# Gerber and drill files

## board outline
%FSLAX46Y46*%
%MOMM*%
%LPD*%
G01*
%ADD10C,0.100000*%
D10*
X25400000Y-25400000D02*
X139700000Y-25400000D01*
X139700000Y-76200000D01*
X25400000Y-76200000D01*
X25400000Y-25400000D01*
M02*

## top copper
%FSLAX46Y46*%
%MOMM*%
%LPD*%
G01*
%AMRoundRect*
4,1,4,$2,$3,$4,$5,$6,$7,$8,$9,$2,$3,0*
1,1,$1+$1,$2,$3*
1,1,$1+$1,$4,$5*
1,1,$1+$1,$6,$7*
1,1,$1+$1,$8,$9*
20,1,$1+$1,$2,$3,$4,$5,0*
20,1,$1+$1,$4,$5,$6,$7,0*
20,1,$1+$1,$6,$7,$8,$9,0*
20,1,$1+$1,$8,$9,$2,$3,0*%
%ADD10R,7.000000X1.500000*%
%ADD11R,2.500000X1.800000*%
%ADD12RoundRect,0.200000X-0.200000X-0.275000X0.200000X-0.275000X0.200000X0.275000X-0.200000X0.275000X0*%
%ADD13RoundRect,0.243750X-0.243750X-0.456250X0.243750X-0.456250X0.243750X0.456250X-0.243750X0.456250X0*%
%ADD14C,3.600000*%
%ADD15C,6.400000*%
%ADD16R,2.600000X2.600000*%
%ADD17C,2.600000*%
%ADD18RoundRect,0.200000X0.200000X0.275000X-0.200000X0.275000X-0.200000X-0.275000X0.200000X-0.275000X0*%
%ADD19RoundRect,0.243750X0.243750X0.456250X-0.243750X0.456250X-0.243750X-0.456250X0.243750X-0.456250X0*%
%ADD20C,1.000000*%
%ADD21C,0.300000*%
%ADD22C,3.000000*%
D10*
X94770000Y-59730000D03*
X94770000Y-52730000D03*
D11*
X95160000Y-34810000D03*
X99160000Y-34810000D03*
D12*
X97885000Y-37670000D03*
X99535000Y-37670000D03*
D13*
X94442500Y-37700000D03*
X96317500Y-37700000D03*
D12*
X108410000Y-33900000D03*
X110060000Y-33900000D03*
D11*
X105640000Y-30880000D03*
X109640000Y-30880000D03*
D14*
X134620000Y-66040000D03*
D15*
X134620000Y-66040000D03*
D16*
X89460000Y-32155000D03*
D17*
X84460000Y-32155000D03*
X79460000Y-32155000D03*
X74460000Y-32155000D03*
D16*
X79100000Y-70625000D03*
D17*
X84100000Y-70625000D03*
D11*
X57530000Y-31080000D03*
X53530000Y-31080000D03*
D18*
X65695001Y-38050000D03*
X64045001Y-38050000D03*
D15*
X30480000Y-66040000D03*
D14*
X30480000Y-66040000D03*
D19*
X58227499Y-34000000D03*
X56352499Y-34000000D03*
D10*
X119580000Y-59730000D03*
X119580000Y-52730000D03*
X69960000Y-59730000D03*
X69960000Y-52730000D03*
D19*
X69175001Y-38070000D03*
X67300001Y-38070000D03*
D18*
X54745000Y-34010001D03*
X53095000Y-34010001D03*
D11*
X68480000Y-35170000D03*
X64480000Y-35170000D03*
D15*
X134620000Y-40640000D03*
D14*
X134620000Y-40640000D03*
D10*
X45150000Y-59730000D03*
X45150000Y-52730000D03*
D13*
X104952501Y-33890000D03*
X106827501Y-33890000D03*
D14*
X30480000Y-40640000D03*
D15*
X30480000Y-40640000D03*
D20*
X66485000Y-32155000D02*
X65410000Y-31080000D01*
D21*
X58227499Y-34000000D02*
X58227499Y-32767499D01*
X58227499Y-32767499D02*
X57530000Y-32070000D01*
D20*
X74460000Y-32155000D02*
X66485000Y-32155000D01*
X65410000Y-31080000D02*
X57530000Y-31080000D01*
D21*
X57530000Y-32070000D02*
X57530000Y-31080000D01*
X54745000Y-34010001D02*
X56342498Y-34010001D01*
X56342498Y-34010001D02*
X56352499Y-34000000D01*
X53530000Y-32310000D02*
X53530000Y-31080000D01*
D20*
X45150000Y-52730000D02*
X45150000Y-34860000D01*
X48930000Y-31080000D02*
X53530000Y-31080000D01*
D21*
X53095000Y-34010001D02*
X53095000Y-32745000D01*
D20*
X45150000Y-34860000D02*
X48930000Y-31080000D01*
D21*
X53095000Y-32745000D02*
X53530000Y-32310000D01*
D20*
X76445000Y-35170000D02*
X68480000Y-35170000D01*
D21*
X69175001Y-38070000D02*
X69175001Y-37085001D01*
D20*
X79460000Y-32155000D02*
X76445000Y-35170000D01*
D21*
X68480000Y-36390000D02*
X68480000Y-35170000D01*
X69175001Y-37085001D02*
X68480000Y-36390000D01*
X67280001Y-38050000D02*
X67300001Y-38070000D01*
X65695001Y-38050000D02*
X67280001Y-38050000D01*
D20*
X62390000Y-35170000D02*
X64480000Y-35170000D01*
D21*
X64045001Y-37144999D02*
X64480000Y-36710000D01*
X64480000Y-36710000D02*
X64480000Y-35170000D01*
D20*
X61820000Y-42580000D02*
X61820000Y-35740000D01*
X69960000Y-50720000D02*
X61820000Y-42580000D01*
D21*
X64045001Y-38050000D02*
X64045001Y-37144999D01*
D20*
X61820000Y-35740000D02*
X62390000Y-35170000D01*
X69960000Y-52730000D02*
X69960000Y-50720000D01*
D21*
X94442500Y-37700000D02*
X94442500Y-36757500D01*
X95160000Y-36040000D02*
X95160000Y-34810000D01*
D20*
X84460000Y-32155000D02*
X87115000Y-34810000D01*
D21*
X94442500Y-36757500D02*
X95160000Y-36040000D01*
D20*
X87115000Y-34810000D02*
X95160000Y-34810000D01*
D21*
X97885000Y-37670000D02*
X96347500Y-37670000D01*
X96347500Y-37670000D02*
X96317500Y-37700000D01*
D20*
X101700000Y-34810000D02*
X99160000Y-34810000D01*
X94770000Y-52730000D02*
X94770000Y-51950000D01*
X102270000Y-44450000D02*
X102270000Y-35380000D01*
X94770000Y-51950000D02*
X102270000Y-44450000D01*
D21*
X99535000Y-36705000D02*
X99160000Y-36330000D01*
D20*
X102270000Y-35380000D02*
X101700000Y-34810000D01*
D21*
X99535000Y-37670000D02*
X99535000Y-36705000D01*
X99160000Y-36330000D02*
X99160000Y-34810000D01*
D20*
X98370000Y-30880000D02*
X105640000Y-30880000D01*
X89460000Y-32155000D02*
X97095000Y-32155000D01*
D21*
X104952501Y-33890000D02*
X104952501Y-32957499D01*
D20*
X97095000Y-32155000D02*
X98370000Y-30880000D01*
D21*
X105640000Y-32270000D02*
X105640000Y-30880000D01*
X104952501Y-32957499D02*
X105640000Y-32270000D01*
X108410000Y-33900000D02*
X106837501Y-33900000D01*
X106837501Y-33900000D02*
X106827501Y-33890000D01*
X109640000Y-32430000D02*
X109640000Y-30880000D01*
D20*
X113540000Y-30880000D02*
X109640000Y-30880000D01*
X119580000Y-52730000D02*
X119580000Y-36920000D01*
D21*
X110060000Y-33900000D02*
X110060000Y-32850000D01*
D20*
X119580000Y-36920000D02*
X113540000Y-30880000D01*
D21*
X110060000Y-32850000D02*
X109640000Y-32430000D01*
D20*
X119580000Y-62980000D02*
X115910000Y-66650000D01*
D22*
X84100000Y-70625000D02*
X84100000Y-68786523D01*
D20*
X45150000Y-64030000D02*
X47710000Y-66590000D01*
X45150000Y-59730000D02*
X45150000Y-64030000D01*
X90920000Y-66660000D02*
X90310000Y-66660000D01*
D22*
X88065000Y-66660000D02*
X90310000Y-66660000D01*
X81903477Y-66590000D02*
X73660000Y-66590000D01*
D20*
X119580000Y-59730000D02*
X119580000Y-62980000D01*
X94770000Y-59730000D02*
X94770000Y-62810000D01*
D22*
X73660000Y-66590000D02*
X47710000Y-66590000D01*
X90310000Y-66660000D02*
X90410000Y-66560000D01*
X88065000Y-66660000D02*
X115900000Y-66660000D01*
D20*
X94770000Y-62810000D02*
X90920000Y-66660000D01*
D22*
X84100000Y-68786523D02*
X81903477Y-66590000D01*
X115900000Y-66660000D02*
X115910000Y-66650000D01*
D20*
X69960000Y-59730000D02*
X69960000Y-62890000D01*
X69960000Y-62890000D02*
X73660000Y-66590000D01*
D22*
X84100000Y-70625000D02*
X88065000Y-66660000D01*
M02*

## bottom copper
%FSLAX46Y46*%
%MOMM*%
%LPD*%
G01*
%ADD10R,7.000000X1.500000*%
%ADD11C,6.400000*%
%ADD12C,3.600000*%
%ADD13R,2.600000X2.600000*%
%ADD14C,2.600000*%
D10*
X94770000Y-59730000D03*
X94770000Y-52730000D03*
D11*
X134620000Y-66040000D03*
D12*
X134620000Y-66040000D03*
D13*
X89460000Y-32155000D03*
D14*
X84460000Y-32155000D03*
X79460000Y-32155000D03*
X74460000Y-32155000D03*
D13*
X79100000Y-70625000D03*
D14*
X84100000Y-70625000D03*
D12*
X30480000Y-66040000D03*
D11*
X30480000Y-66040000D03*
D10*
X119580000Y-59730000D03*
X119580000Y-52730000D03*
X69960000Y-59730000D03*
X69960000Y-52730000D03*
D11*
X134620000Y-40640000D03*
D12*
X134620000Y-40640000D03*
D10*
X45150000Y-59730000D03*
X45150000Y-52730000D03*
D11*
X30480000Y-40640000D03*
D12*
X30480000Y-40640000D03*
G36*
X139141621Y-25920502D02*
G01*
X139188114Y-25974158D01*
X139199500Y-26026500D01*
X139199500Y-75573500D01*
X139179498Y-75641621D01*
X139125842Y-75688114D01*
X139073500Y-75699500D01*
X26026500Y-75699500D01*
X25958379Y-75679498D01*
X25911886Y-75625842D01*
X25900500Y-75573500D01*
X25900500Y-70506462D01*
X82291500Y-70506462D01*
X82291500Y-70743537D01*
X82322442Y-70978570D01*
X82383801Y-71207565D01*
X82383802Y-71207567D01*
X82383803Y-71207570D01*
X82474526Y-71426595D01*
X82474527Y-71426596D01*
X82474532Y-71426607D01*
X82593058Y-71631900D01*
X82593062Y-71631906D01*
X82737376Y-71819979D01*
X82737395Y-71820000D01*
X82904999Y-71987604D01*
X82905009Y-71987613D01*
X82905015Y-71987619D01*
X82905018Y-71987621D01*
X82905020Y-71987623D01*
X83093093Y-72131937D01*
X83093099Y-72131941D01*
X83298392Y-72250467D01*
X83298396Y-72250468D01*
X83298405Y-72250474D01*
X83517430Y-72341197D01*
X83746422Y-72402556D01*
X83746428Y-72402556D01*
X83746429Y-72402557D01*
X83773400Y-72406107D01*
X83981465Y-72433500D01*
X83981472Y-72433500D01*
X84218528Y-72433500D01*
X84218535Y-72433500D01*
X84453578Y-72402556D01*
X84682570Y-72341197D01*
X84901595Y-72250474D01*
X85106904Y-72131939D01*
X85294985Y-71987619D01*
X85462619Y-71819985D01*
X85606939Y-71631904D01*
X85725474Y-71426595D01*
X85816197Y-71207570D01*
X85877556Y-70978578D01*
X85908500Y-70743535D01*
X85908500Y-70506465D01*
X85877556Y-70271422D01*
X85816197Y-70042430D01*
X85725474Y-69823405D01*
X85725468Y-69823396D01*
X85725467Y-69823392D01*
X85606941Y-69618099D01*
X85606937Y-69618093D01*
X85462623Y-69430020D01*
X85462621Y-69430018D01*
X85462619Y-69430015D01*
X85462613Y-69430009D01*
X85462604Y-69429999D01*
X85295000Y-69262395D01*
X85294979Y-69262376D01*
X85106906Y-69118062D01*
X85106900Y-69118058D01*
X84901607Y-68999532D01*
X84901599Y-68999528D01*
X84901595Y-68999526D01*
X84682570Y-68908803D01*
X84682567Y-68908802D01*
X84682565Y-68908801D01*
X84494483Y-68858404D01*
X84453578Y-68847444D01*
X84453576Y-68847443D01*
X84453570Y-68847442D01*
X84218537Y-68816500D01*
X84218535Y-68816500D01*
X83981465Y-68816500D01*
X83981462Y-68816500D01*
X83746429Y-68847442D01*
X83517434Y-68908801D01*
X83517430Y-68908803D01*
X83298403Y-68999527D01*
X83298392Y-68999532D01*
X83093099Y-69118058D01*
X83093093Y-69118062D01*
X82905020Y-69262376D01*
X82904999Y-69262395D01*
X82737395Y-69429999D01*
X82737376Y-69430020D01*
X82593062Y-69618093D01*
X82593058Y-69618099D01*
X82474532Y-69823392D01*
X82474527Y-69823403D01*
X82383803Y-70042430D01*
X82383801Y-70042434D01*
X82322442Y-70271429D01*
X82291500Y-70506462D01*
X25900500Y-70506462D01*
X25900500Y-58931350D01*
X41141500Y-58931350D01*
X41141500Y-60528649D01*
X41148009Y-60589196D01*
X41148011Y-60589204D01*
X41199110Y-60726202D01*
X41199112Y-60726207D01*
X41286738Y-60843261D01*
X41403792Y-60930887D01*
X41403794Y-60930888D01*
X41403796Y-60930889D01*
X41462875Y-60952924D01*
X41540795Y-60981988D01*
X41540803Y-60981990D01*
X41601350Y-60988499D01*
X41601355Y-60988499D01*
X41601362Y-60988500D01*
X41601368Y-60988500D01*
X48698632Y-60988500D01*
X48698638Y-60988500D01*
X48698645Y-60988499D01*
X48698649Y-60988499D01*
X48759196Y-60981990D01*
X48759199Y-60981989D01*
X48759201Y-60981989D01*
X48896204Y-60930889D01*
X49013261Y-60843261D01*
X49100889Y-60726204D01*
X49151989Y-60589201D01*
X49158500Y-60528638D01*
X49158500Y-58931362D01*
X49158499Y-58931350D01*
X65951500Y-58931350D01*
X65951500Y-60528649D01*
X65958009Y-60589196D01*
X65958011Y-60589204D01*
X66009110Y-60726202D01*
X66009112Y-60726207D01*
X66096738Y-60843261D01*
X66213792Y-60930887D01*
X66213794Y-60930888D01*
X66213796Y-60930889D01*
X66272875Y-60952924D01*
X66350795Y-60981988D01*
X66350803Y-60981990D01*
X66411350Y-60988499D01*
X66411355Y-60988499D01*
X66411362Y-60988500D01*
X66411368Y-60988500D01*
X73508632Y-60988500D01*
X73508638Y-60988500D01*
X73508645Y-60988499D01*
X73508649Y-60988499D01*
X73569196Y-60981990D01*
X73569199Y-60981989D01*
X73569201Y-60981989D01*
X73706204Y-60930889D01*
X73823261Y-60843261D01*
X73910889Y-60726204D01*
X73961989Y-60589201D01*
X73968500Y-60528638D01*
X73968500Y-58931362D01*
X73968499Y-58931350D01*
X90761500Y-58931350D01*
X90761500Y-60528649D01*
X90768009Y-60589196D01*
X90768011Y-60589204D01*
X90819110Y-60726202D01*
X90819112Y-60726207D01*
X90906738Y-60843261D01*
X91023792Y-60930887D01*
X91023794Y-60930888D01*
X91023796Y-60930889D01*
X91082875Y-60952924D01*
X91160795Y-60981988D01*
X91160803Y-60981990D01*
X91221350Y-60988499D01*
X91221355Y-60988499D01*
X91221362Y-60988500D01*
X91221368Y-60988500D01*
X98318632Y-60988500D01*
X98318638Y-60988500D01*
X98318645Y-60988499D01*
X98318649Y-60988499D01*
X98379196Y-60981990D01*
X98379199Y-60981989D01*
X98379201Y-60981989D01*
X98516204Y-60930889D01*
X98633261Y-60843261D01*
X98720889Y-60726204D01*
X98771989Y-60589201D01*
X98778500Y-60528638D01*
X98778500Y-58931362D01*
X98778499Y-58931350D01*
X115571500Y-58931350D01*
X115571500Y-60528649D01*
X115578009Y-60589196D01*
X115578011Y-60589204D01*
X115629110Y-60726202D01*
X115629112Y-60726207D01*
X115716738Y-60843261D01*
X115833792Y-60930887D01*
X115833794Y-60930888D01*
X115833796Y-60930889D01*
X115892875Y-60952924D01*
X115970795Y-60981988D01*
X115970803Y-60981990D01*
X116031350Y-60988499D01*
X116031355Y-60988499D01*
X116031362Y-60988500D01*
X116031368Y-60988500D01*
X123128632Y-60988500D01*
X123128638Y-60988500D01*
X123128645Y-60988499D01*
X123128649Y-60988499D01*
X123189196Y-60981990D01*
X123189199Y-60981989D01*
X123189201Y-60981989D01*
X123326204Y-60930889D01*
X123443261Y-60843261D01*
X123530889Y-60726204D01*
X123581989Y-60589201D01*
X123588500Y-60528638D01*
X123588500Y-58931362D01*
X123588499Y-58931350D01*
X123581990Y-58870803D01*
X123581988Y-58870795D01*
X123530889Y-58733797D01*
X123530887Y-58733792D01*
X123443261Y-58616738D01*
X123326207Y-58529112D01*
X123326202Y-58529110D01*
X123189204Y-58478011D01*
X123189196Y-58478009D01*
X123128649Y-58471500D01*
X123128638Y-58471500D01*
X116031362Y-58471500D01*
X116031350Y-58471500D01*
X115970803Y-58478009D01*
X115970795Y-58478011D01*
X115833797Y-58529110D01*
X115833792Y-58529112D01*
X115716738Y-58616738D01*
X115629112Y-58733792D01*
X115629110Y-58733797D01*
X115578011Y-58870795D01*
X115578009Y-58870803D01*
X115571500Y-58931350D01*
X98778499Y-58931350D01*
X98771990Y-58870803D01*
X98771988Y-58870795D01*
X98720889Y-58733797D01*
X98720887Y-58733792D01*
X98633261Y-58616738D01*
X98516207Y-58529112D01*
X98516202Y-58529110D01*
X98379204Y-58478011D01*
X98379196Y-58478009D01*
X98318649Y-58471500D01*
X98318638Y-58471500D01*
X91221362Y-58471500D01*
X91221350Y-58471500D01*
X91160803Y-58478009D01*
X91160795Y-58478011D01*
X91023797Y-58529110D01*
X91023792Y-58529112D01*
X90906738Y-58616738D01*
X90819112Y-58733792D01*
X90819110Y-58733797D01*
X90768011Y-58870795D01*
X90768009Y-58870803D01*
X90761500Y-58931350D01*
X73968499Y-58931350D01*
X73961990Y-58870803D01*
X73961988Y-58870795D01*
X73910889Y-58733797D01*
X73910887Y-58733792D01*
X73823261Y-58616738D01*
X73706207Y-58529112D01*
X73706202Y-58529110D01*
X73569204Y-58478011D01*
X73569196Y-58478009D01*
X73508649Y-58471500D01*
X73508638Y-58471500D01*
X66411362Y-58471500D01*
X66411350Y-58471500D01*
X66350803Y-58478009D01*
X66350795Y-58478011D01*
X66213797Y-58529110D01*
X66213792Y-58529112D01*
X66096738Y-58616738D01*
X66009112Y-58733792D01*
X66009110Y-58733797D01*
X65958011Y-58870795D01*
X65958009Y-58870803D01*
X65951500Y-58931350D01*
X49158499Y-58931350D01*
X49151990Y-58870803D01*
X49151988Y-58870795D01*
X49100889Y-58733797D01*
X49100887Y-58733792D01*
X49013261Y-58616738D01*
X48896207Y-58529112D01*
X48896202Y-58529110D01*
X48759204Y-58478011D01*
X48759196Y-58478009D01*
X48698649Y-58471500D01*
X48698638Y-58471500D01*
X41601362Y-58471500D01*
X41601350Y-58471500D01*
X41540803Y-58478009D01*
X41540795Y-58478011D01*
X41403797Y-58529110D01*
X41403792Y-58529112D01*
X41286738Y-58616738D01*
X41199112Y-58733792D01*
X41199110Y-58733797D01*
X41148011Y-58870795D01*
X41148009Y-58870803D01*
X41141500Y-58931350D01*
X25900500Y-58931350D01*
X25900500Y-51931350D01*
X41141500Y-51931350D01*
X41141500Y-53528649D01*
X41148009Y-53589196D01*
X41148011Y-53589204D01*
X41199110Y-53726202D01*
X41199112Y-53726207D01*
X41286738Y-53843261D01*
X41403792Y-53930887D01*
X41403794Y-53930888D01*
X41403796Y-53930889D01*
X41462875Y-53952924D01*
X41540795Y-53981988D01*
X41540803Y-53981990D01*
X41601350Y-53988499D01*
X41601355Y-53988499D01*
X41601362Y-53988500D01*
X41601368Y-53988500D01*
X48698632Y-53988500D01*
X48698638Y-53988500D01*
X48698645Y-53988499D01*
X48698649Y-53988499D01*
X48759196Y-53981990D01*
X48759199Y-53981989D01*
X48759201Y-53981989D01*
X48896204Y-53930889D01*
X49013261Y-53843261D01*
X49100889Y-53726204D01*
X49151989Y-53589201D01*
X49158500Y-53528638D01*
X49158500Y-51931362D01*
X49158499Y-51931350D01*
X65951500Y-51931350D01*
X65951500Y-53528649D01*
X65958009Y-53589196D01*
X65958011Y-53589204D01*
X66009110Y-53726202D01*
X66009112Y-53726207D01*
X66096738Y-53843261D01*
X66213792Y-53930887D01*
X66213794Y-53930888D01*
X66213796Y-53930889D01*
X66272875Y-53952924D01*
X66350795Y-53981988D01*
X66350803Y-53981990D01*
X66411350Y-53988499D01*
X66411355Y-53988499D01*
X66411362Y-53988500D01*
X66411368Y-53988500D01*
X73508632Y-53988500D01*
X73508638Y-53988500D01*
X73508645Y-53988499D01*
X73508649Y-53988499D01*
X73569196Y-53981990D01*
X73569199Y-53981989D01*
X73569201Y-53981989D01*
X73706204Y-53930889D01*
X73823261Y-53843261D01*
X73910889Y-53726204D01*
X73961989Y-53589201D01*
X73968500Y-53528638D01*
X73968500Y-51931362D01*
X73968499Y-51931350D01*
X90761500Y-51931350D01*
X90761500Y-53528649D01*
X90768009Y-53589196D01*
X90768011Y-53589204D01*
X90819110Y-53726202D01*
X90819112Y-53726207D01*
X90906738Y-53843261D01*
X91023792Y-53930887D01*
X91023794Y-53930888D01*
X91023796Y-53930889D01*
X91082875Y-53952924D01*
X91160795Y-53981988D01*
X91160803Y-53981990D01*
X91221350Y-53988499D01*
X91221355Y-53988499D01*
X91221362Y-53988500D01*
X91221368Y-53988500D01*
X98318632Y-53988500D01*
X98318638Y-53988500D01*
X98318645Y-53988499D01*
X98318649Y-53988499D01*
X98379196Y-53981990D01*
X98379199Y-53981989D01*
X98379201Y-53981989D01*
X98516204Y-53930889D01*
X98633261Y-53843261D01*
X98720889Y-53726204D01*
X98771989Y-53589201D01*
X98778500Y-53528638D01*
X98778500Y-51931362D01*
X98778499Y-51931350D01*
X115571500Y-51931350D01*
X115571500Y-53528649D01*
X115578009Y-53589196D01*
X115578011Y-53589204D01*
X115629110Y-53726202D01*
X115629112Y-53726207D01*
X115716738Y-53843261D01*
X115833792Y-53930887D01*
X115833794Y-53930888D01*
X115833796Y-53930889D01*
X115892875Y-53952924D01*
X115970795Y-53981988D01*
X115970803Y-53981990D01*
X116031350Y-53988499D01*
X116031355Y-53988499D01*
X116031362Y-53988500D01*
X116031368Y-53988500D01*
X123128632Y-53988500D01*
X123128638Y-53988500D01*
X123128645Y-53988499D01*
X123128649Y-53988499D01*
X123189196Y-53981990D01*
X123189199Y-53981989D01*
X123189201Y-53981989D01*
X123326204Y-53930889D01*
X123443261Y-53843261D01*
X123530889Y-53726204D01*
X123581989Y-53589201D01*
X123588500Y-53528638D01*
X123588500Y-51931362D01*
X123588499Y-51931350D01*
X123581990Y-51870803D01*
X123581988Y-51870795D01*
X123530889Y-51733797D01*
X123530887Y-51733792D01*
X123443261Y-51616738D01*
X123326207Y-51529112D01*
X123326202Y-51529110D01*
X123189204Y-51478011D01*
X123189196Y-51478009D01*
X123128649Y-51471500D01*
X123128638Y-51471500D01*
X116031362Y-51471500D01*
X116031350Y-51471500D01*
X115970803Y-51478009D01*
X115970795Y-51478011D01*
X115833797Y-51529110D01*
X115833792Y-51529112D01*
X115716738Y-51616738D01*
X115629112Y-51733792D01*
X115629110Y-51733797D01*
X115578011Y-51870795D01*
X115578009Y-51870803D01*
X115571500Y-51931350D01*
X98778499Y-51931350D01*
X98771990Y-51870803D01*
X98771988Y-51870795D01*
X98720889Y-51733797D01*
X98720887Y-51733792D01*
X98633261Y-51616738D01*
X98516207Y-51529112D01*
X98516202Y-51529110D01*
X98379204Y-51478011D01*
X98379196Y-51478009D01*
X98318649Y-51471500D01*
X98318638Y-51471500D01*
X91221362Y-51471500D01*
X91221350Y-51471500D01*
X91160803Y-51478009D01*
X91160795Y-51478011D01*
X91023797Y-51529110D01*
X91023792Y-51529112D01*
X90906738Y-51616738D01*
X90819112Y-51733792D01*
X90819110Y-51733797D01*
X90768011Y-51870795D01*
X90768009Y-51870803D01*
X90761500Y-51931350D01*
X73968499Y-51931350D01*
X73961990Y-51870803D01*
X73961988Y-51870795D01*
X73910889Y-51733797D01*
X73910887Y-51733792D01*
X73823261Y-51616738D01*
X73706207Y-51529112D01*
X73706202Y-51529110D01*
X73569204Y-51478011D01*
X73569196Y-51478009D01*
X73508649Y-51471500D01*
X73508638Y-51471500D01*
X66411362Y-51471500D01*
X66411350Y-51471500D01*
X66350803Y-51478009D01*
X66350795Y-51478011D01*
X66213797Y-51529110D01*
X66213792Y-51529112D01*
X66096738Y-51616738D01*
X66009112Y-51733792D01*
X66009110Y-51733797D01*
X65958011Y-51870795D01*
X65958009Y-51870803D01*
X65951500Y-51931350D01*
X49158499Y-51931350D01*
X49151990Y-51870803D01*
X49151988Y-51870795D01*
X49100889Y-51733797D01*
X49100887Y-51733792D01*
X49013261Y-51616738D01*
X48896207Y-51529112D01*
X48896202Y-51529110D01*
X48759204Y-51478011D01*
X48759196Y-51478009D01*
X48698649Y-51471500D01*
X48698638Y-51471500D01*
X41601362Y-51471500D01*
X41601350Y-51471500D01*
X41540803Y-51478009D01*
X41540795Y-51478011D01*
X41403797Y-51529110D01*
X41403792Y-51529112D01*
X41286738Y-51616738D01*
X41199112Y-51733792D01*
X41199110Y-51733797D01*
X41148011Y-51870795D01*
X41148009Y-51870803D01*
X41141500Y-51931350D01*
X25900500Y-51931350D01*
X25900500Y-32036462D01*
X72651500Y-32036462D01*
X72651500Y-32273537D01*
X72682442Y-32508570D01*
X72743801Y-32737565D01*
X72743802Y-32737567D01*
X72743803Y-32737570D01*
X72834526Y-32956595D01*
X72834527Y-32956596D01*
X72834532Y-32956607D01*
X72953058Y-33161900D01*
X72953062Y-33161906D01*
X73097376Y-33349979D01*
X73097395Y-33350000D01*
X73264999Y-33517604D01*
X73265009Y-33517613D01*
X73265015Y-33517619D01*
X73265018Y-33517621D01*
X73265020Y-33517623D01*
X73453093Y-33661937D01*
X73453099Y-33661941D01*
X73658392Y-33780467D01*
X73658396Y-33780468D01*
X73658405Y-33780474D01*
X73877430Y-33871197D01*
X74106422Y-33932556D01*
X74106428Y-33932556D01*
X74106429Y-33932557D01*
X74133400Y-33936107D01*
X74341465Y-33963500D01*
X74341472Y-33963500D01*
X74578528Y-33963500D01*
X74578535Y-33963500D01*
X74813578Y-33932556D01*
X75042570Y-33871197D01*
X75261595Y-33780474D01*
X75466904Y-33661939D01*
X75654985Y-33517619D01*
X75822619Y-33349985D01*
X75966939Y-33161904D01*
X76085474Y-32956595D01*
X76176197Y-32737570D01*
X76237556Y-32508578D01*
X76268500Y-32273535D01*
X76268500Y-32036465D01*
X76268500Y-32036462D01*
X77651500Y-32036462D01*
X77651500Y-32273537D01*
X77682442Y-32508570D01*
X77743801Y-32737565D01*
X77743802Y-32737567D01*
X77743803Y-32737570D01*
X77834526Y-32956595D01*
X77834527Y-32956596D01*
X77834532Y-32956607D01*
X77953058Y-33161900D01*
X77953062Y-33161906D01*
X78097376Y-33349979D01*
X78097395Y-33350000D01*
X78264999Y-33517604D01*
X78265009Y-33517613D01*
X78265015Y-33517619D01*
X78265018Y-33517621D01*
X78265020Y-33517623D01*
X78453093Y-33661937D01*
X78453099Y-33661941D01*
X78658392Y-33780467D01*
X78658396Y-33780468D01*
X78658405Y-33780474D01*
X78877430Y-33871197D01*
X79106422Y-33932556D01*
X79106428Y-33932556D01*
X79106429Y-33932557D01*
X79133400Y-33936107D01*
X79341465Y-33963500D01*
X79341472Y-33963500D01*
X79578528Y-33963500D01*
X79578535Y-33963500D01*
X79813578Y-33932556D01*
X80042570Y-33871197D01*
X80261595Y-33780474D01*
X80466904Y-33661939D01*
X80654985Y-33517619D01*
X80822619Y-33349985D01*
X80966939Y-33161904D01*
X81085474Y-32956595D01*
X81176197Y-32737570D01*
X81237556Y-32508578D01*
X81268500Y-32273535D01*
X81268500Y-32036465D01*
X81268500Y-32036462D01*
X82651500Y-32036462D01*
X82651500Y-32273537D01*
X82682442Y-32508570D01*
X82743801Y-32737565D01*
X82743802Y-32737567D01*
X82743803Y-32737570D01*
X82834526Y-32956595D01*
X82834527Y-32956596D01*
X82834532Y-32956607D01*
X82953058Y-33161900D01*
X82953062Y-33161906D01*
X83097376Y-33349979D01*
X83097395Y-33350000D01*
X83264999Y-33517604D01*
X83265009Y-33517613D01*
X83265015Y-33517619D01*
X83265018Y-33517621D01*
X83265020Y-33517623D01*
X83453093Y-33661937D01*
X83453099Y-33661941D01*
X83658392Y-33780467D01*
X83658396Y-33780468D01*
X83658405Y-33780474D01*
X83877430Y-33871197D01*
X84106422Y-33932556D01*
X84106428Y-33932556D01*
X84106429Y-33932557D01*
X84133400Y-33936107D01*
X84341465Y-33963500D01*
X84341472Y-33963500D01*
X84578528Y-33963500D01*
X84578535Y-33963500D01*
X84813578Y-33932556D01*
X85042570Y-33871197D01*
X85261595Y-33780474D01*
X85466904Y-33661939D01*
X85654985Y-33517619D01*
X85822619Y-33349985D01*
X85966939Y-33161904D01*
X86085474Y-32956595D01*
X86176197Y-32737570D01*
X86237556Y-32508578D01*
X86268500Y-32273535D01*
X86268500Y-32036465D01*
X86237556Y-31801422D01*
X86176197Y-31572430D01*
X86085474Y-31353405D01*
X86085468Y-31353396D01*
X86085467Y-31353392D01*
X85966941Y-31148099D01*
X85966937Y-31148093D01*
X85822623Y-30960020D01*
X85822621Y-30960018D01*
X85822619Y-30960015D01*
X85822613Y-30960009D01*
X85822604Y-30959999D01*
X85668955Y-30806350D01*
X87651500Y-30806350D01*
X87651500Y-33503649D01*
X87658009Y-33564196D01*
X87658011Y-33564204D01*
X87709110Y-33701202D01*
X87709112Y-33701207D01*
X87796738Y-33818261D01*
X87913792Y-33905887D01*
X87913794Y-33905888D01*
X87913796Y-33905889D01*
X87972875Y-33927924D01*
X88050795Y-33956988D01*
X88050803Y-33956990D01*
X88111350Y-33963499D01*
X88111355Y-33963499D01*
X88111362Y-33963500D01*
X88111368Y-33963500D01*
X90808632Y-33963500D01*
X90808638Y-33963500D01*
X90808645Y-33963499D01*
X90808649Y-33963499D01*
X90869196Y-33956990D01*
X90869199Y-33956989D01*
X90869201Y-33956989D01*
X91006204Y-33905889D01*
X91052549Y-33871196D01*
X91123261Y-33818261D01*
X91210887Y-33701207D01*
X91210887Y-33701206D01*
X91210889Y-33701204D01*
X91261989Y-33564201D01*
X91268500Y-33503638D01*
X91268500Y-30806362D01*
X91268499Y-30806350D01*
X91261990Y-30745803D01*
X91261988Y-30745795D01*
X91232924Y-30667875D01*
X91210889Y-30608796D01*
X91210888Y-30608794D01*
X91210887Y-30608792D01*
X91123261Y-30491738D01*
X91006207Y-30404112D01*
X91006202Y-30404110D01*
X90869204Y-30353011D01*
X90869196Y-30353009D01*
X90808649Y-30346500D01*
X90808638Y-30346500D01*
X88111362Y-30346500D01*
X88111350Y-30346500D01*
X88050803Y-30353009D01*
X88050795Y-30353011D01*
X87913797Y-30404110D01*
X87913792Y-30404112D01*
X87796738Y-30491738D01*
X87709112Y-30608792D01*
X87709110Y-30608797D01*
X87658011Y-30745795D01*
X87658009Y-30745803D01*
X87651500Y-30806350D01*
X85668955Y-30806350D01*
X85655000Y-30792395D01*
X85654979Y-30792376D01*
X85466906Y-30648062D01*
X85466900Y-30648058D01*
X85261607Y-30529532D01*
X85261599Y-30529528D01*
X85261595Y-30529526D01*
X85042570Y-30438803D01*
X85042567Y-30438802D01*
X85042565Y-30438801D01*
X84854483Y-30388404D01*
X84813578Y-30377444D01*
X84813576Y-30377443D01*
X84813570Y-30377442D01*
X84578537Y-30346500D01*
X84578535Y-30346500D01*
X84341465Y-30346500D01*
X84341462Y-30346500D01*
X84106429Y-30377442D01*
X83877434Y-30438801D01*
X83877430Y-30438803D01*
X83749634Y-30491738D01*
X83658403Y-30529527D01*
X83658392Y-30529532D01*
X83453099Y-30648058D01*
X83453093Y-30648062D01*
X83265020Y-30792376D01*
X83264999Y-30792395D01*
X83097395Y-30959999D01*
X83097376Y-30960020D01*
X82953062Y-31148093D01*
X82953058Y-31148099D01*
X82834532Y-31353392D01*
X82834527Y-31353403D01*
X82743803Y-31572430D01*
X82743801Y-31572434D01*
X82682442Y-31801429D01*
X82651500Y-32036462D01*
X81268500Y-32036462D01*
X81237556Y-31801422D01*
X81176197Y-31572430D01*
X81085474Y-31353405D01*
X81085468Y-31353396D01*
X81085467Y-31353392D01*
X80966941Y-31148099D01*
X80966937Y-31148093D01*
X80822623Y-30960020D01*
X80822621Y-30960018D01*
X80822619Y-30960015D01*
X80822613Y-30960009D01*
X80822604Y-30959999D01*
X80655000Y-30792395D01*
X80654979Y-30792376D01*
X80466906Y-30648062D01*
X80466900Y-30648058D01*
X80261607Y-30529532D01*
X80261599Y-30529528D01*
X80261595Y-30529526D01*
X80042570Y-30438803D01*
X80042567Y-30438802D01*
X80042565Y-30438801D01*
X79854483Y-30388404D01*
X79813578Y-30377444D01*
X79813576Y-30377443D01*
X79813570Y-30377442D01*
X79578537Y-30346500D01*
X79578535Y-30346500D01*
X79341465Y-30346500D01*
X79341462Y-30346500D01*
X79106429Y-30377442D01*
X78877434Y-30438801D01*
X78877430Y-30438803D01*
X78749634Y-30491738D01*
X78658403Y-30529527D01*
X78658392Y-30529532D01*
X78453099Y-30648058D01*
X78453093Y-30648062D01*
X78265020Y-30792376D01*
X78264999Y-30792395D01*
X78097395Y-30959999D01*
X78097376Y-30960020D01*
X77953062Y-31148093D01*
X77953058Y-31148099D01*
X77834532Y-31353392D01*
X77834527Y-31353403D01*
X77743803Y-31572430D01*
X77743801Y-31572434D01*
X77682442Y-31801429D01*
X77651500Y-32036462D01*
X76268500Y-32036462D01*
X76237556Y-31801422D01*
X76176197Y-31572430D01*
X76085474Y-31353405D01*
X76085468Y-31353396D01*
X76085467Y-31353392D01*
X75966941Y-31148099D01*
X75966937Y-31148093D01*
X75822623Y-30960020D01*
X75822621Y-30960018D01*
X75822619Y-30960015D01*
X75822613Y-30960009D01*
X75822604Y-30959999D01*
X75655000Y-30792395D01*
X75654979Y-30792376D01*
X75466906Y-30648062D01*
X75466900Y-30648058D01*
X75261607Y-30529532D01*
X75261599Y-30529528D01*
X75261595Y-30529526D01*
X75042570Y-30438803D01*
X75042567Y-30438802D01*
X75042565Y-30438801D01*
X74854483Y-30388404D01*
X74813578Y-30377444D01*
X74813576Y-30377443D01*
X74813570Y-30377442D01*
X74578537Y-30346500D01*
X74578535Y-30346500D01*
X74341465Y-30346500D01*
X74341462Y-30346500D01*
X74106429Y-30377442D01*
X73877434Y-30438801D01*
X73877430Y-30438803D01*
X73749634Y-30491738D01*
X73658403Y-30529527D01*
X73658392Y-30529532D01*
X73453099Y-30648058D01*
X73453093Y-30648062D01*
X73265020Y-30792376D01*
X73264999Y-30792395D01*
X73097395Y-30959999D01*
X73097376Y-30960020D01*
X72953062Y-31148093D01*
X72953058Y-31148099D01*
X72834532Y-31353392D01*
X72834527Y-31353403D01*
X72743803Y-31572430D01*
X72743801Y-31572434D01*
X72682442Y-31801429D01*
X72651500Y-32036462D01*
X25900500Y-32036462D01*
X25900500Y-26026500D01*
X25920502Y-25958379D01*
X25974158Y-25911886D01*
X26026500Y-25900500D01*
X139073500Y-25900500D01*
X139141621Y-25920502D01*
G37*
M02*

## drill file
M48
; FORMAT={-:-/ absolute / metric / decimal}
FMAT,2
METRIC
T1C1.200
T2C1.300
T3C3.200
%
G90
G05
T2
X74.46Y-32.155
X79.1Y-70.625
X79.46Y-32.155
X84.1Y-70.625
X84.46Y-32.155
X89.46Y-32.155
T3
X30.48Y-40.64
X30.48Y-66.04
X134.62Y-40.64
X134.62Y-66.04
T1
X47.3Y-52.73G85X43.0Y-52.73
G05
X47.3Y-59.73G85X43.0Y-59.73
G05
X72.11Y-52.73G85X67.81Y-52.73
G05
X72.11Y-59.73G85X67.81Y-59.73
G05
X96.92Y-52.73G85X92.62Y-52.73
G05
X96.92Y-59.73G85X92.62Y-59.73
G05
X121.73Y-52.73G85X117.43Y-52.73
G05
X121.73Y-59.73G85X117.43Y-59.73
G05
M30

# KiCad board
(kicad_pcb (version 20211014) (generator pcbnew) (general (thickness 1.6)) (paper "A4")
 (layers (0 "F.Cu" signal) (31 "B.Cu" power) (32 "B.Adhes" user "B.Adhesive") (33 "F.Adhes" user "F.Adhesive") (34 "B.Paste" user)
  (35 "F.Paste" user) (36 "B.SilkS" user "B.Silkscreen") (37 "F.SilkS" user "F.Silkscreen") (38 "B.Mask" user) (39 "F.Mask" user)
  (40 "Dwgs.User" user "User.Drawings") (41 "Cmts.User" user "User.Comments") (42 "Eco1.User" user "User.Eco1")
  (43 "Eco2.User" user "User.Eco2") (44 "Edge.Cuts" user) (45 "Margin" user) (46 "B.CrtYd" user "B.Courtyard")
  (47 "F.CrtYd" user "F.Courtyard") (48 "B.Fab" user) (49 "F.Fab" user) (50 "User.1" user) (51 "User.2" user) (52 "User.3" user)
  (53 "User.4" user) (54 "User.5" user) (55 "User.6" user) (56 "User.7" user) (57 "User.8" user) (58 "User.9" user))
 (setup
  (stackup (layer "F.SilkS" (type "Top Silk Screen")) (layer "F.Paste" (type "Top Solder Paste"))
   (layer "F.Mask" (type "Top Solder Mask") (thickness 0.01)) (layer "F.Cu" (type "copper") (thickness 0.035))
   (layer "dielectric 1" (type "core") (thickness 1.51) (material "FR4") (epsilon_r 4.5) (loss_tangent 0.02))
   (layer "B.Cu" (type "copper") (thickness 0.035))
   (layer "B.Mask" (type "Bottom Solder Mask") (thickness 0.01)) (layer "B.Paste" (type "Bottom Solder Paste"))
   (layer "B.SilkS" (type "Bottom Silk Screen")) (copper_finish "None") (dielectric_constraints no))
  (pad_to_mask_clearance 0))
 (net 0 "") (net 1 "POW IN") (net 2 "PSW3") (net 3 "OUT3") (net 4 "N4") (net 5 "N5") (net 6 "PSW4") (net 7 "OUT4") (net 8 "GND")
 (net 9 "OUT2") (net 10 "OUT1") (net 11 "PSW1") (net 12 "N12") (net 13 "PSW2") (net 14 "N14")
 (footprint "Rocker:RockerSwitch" (layer "F.Cu") (at 94.77 52.73 180)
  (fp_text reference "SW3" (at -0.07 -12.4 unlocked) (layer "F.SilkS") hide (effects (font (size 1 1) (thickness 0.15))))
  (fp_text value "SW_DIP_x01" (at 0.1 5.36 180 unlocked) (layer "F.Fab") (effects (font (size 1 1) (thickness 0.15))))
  (pad "1" thru_hole rect (at 0 -7 180) (size 7 1.5) (drill oval 5.5 1.2) (layers *.Cu *.Mask "B.Adhes") (remove_unused_layers)
   (keep_end_layers) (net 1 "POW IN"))
  (pad "2" thru_hole rect (at 0 0 180) (size 7 1.5) (drill oval 5.5 1.2) (layers *.Cu *.Mask) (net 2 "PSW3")))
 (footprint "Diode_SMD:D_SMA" (layer "F.Cu") (at 97.16 34.81)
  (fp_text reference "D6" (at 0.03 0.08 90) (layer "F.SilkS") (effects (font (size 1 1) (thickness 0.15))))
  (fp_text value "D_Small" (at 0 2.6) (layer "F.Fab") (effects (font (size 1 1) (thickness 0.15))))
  (pad "1" smd rect (at -2 0) (size 2.5 1.8) (layers "F.Cu" "F.Paste" "F.Mask") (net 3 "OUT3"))
  (pad "2" smd rect (at 2 0) (size 2.5 1.8) (layers "F.Cu" "F.Paste" "F.Mask") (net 2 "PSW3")))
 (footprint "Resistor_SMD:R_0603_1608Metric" (layer "F.Cu") (at 98.71 37.67)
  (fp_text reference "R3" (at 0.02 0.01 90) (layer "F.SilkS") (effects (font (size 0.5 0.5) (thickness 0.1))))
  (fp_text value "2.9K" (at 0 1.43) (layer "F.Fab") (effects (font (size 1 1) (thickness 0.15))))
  (pad "1" smd roundrect (at -0.825 0) (size 0.8 0.95) (layers "F.Cu" "F.Paste" "F.Mask") (roundrect_rratio 0.25) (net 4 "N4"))
  (pad "2" smd roundrect (at 0.825 0) (size 0.8 0.95) (layers "F.Cu" "F.Paste" "F.Mask") (roundrect_rratio 0.25) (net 2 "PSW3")))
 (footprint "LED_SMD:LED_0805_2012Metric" (layer "F.Cu") (at 95.38 37.7)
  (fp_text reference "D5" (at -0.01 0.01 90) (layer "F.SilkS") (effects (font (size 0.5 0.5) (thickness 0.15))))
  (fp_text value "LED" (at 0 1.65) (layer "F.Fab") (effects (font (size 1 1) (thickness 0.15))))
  (pad "1" smd roundrect (at -0.9375 0) (size 0.975 1.4) (layers "F.Cu" "F.Paste" "F.Mask") (roundrect_rratio 0.25) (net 3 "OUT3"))
  (pad "2" smd roundrect (at 0.9375 0) (size 0.975 1.4) (layers "F.Cu" "F.Paste" "F.Mask") (roundrect_rratio 0.25) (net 4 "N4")))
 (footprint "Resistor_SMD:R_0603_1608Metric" (layer "F.Cu") (at 109.235 33.9)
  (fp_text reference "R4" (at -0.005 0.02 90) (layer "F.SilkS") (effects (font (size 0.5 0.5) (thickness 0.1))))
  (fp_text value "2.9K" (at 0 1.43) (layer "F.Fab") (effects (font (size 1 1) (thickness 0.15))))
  (pad "1" smd roundrect (at -0.825 0) (size 0.8 0.95) (layers "F.Cu" "F.Paste" "F.Mask") (roundrect_rratio 0.25) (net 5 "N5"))
  (pad "2" smd roundrect (at 0.825 0) (size 0.8 0.95) (layers "F.Cu" "F.Paste" "F.Mask") (roundrect_rratio 0.25) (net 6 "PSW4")))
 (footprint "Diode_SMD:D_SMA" (layer "F.Cu") (at 107.64 30.88)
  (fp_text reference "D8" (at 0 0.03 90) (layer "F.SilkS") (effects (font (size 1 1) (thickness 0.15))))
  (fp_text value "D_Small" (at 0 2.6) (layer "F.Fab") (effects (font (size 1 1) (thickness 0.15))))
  (pad "1" smd rect (at -2 0) (size 2.5 1.8) (layers "F.Cu" "F.Paste" "F.Mask") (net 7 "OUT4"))
  (pad "2" smd rect (at 2 0) (size 2.5 1.8) (layers "F.Cu" "F.Paste" "F.Mask") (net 6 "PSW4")))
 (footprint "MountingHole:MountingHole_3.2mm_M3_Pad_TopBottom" (layer "F.Cu") (at 134.62 66.04)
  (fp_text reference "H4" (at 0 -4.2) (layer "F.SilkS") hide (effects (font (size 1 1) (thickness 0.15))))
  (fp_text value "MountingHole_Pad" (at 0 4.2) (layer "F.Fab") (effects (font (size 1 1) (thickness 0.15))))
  (pad "1" connect circle (at 0 0) (size 6.4 6.4) (layers "B.Cu" "B.Mask") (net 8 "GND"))
  (pad "1" thru_hole circle (at 0 0) (size 3.6 3.6) (drill 3.2) (layers *.Cu *.Mask) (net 8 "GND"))
  (pad "1" connect circle (at 0 0) (size 6.4 6.4) (layers "F.Cu" "F.Mask") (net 8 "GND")))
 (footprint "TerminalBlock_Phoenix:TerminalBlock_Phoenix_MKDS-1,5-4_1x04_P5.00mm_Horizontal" (layer "F.Cu") (at 89.46 32.155 180)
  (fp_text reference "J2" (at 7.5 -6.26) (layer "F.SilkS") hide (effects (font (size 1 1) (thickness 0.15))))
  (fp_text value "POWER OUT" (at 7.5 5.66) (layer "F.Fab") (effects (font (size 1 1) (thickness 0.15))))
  (pad "1" thru_hole rect (at 0 0 180) (size 2.6 2.6) (drill 1.3) (layers *.Cu *.Mask) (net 7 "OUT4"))
  (pad "2" thru_hole circle (at 5 0 180) (size 2.6 2.6) (drill 1.3) (layers *.Cu *.Mask) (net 3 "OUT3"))
  (pad "3" thru_hole circle (at 10 0 180) (size 2.6 2.6) (drill 1.3) (layers *.Cu *.Mask) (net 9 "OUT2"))
  (pad "4" thru_hole circle (at 15 0 180) (size 2.6 2.6) (drill 1.3) (layers *.Cu *.Mask) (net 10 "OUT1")))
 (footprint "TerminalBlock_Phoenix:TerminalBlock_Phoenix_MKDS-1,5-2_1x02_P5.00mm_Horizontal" (layer "F.Cu") (at 79.1 70.625)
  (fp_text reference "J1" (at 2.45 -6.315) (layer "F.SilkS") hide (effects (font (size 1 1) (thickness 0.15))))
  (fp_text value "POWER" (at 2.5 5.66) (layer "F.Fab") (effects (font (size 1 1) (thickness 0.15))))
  (pad "1" thru_hole rect (at 0 0) (size 2.6 2.6) (drill 1.3) (layers *.Cu *.Mask) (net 8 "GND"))
  (pad "2" thru_hole circle (at 5 0) (size 2.6 2.6) (drill 1.3) (layers *.Cu *.Mask) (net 1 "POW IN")))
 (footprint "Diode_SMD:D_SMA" (layer "F.Cu") (at 55.53 31.08 180)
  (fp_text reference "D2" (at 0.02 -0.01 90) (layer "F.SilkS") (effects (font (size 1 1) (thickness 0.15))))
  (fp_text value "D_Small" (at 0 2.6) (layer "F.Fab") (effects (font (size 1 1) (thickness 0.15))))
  (pad "1" smd rect (at -2 0 180) (size 2.5 1.8) (layers "F.Cu" "F.Paste" "F.Mask") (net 10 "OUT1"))
  (pad "2" smd rect (at 2 0 180) (size 2.5 1.8) (layers "F.Cu" "F.Paste" "F.Mask") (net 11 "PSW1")))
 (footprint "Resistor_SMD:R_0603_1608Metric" (layer "F.Cu") (at 64.870001 38.05 180)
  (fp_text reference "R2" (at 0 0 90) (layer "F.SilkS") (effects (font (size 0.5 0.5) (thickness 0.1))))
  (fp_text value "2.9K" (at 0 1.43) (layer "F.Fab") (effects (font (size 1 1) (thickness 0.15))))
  (pad "1" smd roundrect (at -0.825 0 180) (size 0.8 0.95) (layers "F.Cu" "F.Paste" "F.Mask") (roundrect_rratio 0.25) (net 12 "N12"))
  (pad "2" smd roundrect (at 0.825 0 180) (size 0.8 0.95) (layers "F.Cu" "F.Paste" "F.Mask") (roundrect_rratio 0.25) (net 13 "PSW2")))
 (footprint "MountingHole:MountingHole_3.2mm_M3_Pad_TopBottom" (layer "F.Cu") (at 30.48 66.04)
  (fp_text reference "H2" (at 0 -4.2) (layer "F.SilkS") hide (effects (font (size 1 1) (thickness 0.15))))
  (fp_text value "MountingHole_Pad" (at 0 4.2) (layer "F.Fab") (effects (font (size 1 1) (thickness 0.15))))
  (pad "1" connect circle (at 0 0) (size 6.4 6.4) (layers "F.Cu" "F.Mask") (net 8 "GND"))
  (pad "1" thru_hole circle (at 0 0) (size 3.6 3.6) (drill 3.2) (layers *.Cu *.Mask) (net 8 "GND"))
  (pad "1" connect circle (at 0 0) (size 6.4 6.4) (layers "B.Cu" "B.Mask") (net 8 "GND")))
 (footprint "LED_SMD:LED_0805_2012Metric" (layer "F.Cu") (at 57.289999 34 180)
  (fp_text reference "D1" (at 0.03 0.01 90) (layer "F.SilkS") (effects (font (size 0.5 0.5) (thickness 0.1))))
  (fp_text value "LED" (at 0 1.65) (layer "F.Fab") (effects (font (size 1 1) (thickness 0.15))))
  (pad "1" smd roundrect (at -0.9375 0 180) (size 0.975 1.4) (layers "F.Cu" "F.Paste" "F.Mask") (roundrect_rratio 0.25) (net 10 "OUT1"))
  (pad "2" smd roundrect (at 0.9375 0 180) (size 0.975 1.4) (layers "F.Cu" "F.Paste" "F.Mask") (roundrect_rratio 0.25) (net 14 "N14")))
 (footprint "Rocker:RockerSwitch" (layer "F.Cu") (at 119.58 52.73 180)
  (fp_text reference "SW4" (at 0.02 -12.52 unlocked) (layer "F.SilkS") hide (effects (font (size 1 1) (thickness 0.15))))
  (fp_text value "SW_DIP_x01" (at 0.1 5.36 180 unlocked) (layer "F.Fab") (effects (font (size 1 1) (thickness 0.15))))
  (pad "1" thru_hole rect (at 0 -7 180) (size 7 1.5) (drill oval 5.5 1.2) (layers *.Cu *.Mask "B.Adhes") (remove_unused_layers)
   (keep_end_layers) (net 1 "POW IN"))
  (pad "2" thru_hole rect (at 0 0 180) (size 7 1.5) (drill oval 5.5 1.2) (layers *.Cu *.Mask) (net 6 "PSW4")))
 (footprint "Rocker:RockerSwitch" (layer "F.Cu") (at 69.96 52.73 180)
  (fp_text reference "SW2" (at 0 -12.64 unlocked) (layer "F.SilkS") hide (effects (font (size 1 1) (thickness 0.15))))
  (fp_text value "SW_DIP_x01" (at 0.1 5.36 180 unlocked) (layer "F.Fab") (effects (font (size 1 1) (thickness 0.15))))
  (pad "1" thru_hole rect (at 0 -7 180) (size 7 1.5) (drill oval 5.5 1.2) (layers *.Cu *.Mask "B.Adhes") (remove_unused_layers)
   (keep_end_layers) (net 1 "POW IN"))
  (pad "2" thru_hole rect (at 0 0 180) (size 7 1.5) (drill oval 5.5 1.2) (layers *.Cu *.Mask) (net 13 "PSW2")))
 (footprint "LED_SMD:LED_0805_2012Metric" (layer "F.Cu") (at 68.237501 38.07 180)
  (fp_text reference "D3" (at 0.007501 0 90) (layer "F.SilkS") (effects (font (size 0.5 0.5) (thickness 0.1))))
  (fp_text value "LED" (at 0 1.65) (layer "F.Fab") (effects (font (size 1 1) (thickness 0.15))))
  (pad "1" smd roundrect (at -0.9375 0 180) (size 0.975 1.4) (layers "F.Cu" "F.Paste" "F.Mask") (roundrect_rratio 0.25) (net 9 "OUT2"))
  (pad "2" smd roundrect (at 0.9375 0 180) (size 0.975 1.4) (layers "F.Cu" "F.Paste" "F.Mask") (roundrect_rratio 0.25) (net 12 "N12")))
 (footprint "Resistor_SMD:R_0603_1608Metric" (layer "F.Cu") (at 53.92 34.010001 180)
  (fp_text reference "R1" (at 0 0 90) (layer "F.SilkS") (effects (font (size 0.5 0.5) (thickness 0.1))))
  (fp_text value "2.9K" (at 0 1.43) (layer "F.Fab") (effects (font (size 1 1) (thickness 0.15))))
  (pad "1" smd roundrect (at -0.825 0 180) (size 0.8 0.95) (layers "F.Cu" "F.Paste" "F.Mask") (roundrect_rratio 0.25) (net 14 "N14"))
  (pad "2" smd roundrect (at 0.825 0 180) (size 0.8 0.95) (layers "F.Cu" "F.Paste" "F.Mask") (roundrect_rratio 0.25) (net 11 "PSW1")))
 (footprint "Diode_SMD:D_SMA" (layer "F.Cu") (at 66.48 35.17 180)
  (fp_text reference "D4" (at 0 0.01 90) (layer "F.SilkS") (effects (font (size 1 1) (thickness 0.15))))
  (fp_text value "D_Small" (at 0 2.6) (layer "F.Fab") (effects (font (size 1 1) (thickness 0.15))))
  (pad "1" smd rect (at -2 0 180) (size 2.5 1.8) (layers "F.Cu" "F.Paste" "F.Mask") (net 9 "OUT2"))
  (pad "2" smd rect (at 2 0 180) (size 2.5 1.8) (layers "F.Cu" "F.Paste" "F.Mask") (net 13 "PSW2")))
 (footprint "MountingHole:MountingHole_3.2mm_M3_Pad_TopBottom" (layer "F.Cu") (at 134.62 40.64)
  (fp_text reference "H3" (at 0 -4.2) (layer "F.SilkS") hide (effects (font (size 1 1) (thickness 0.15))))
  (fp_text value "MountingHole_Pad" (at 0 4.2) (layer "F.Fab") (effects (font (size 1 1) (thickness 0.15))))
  (pad "1" connect circle (at 0 0) (size 6.4 6.4) (layers "F.Cu" "F.Mask") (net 8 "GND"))
  (pad "1" connect circle (at 0 0) (size 6.4 6.4) (layers "B.Cu" "B.Mask") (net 8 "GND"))
  (pad "1" thru_hole circle (at 0 0) (size 3.6 3.6) (drill 3.2) (layers *.Cu *.Mask) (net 8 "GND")))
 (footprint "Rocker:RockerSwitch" (layer "F.Cu") (at 45.15 52.73 180)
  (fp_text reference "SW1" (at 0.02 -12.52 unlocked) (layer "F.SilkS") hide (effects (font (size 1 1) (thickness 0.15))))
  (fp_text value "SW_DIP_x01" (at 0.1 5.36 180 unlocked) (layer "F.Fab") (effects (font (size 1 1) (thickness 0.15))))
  (pad "1" thru_hole rect (at 0 -7 180) (size 7 1.5) (drill oval 5.5 1.2) (layers *.Cu *.Mask "B.Adhes") (remove_unused_layers)
   (keep_end_layers) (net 1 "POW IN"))
  (pad "2" thru_hole rect (at 0 0 180) (size 7 1.5) (drill oval 5.5 1.2) (layers *.Cu *.Mask) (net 11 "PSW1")))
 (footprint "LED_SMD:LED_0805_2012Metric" (layer "F.Cu") (at 105.890001 33.89)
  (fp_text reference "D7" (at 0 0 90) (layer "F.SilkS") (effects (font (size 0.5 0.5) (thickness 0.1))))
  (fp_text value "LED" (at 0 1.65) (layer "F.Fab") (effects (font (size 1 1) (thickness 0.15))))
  (pad "1" smd roundrect (at -0.9375 0) (size 0.975 1.4) (layers "F.Cu" "F.Paste" "F.Mask") (roundrect_rratio 0.25) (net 7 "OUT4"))
  (pad "2" smd roundrect (at 0.9375 0) (size 0.975 1.4) (layers "F.Cu" "F.Paste" "F.Mask") (roundrect_rratio 0.25) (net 5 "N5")))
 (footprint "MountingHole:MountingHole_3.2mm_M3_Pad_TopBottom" (layer "F.Cu") (at 30.48 40.64)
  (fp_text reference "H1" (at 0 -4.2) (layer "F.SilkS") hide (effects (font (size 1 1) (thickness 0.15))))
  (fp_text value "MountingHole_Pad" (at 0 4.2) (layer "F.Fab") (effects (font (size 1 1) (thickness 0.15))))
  (pad "1" connect circle (at 0 0) (size 6.4 6.4) (layers "B.Cu" "B.Mask") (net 8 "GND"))
  (pad "1" thru_hole circle (at 0 0) (size 3.6 3.6) (drill 3.2) (layers *.Cu *.Mask) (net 8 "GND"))
  (pad "1" connect circle (at 0 0) (size 6.4 6.4) (layers "F.Cu" "F.Mask") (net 8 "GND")))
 (gr_rect (start 25.4 25.4) (end 139.7 76.2) (layer "Edge.Cuts") (width 0.1) (fill none))
 (segment (start 66.485 32.155) (end 65.41 31.08) (width 1) (layer "F.Cu") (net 10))
 (segment (start 58.227499 34) (end 58.227499 32.767499) (width 0.3) (layer "F.Cu") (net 10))
 (segment (start 58.227499 32.767499) (end 57.53 32.07) (width 0.3) (layer "F.Cu") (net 10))
 (segment (start 74.46 32.155) (end 66.485 32.155) (width 1) (layer "F.Cu") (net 10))
 (segment (start 65.41 31.08) (end 57.53 31.08) (width 1) (layer "F.Cu") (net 10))
 (segment (start 57.53 32.07) (end 57.53 31.08) (width 0.3) (layer "F.Cu") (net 10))
 (segment (start 54.745 34.010001) (end 56.342498 34.010001) (width 0.3) (layer "F.Cu") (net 14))
 (segment (start 56.342498 34.010001) (end 56.352499 34) (width 0.3) (layer "F.Cu") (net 14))
 (segment (start 53.53 32.31) (end 53.53 31.08) (width 0.3) (layer "F.Cu") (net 11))
 (segment (start 45.15 52.73) (end 45.15 34.86) (width 1) (layer "F.Cu") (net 11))
 (segment (start 48.93 31.08) (end 53.53 31.08) (width 1) (layer "F.Cu") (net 11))
 (segment (start 53.095 34.010001) (end 53.095 32.745) (width 0.3) (layer "F.Cu") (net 11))
 (segment (start 45.15 34.86) (end 48.93 31.08) (width 1) (layer "F.Cu") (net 11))
 (segment (start 53.095 32.745) (end 53.53 32.31) (width 0.3) (layer "F.Cu") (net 11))
 (segment (start 76.445 35.17) (end 68.48 35.17) (width 1) (layer "F.Cu") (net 9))
 (segment (start 69.175001 38.07) (end 69.175001 37.085001) (width 0.3) (layer "F.Cu") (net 9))
 (segment (start 79.46 32.155) (end 76.445 35.17) (width 1) (layer "F.Cu") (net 9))
 (segment (start 68.48 36.39) (end 68.48 35.17) (width 0.3) (layer "F.Cu") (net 9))
 (segment (start 69.175001 37.085001) (end 68.48 36.39) (width 0.3) (layer "F.Cu") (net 9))
 (segment (start 67.280001 38.05) (end 67.300001 38.07) (width 0.3) (layer "F.Cu") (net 12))
 (segment (start 65.695001 38.05) (end 67.280001 38.05) (width 0.3) (layer "F.Cu") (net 12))
 (segment (start 62.39 35.17) (end 64.48 35.17) (width 1) (layer "F.Cu") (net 13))
 (segment (start 64.045001 37.144999) (end 64.48 36.71) (width 0.3) (layer "F.Cu") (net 13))
 (segment (start 64.48 36.71) (end 64.48 35.17) (width 0.3) (layer "F.Cu") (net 13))
 (segment (start 61.82 42.58) (end 61.82 35.74) (width 1) (layer "F.Cu") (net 13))
 (segment (start 69.96 50.72) (end 61.82 42.58) (width 1) (layer "F.Cu") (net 13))
 (segment (start 64.045001 38.05) (end 64.045001 37.144999) (width 0.3) (layer "F.Cu") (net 13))
 (segment (start 61.82 35.74) (end 62.39 35.17) (width 1) (layer "F.Cu") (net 13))
 (segment (start 69.96 52.73) (end 69.96 50.72) (width 1) (layer "F.Cu") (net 13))
 (segment (start 94.4425 37.7) (end 94.4425 36.7575) (width 0.3) (layer "F.Cu") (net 3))
 (segment (start 95.16 36.04) (end 95.16 34.81) (width 0.3) (layer "F.Cu") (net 3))
 (segment (start 84.46 32.155) (end 87.115 34.81) (width 1) (layer "F.Cu") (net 3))
 (segment (start 94.4425 36.7575) (end 95.16 36.04) (width 0.3) (layer "F.Cu") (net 3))
 (segment (start 87.115 34.81) (end 95.16 34.81) (width 1) (layer "F.Cu") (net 3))
 (segment (start 97.885 37.67) (end 96.3475 37.67) (width 0.3) (layer "F.Cu") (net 4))
 (segment (start 96.3475 37.67) (end 96.3175 37.7) (width 0.3) (layer "F.Cu") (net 4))
 (segment (start 101.7 34.81) (end 99.16 34.81) (width 1) (layer "F.Cu") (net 2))
 (segment (start 94.77 52.73) (end 94.77 51.95) (width 1) (layer "F.Cu") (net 2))
 (segment (start 102.27 44.45) (end 102.27 35.38) (width 1) (layer "F.Cu") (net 2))
 (segment (start 94.77 51.95) (end 102.27 44.45) (width 1) (layer "F.Cu") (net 2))
 (segment (start 99.535 36.705) (end 99.16 36.33) (width 0.3) (layer "F.Cu") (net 2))
 (segment (start 102.27 35.38) (end 101.7 34.81) (width 1) (layer "F.Cu") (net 2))
 (segment (start 99.535 37.67) (end 99.535 36.705) (width 0.3) (layer "F.Cu") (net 2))
 (segment (start 99.16 36.33) (end 99.16 34.81) (width 0.3) (layer "F.Cu") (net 2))
 (segment (start 98.37 30.88) (end 105.64 30.88) (width 1) (layer "F.Cu") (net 7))
 (segment (start 89.46 32.155) (end 97.095 32.155) (width 1) (layer "F.Cu") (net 7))
 (segment (start 104.952501 33.89) (end 104.952501 32.957499) (width 0.3) (layer "F.Cu") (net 7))
 (segment (start 97.095 32.155) (end 98.37 30.88) (width 1) (layer "F.Cu") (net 7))
 (segment (start 105.64 32.27) (end 105.64 30.88) (width 0.3) (layer "F.Cu") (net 7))
 (segment (start 104.952501 32.957499) (end 105.64 32.27) (width 0.3) (layer "F.Cu") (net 7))
 (segment (start 108.41 33.9) (end 106.837501 33.9) (width 0.3) (layer "F.Cu") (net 5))
 (segment (start 106.837501 33.9) (end 106.827501 33.89) (width 0.3) (layer "F.Cu") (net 5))
 (segment (start 109.64 32.43) (end 109.64 30.88) (width 0.3) (layer "F.Cu") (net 6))
 (segment (start 113.54 30.88) (end 109.64 30.88) (width 1) (layer "F.Cu") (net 6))
 (segment (start 119.58 52.73) (end 119.58 36.92) (width 1) (layer "F.Cu") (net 6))
 (segment (start 110.06 33.9) (end 110.06 32.85) (width 0.3) (layer "F.Cu") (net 6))
 (segment (start 119.58 36.92) (end 113.54 30.88) (width 1) (layer "F.Cu") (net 6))
 (segment (start 110.06 32.85) (end 109.64 32.43) (width 0.3) (layer "F.Cu") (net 6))
 (segment (start 119.58 62.98) (end 115.91 66.65) (width 1) (layer "F.Cu") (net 1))
 (segment (start 84.1 70.625) (end 84.1 68.786523) (width 3) (layer "F.Cu") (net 1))
 (segment (start 45.15 64.03) (end 47.71 66.59) (width 1) (layer "F.Cu") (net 1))
 (segment (start 45.15 59.73) (end 45.15 64.03) (width 1) (layer "F.Cu") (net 1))
 (segment (start 90.92 66.66) (end 90.31 66.66) (width 1) (layer "F.Cu") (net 1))
 (segment (start 88.065 66.66) (end 90.31 66.66) (width 3) (layer "F.Cu") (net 1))
 (segment (start 81.903477 66.59) (end 73.66 66.59) (width 3) (layer "F.Cu") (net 1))
 (segment (start 119.58 59.73) (end 119.58 62.98) (width 1) (layer "F.Cu") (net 1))
 (segment (start 94.77 59.73) (end 94.77 62.81) (width 1) (layer "F.Cu") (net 1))
 (segment (start 73.66 66.59) (end 47.71 66.59) (width 3) (layer "F.Cu") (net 1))
 (segment (start 90.31 66.66) (end 90.41 66.56) (width 3) (layer "F.Cu") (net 1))
 (segment (start 88.065 66.66) (end 115.9 66.66) (width 3) (layer "F.Cu") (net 1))
 (segment (start 94.77 62.81) (end 90.92 66.66) (width 1) (layer "F.Cu") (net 1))
 (segment (start 84.1 68.786523) (end 81.903477 66.59) (width 3) (layer "F.Cu") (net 1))
 (segment (start 115.9 66.66) (end 115.91 66.65) (width 3) (layer "F.Cu") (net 1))
 (segment (start 69.96 59.73) (end 69.96 62.89) (width 1) (layer "F.Cu") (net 1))
 (segment (start 69.96 62.89) (end 73.66 66.59) (width 1) (layer "F.Cu") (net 1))
 (segment (start 84.1 70.625) (end 88.065 66.66) (width 3) (layer "F.Cu") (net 1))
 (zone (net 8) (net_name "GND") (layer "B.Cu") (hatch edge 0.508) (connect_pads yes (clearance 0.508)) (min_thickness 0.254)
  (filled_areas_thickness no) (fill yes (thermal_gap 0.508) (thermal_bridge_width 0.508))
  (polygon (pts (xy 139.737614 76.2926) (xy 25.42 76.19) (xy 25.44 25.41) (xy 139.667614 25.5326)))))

